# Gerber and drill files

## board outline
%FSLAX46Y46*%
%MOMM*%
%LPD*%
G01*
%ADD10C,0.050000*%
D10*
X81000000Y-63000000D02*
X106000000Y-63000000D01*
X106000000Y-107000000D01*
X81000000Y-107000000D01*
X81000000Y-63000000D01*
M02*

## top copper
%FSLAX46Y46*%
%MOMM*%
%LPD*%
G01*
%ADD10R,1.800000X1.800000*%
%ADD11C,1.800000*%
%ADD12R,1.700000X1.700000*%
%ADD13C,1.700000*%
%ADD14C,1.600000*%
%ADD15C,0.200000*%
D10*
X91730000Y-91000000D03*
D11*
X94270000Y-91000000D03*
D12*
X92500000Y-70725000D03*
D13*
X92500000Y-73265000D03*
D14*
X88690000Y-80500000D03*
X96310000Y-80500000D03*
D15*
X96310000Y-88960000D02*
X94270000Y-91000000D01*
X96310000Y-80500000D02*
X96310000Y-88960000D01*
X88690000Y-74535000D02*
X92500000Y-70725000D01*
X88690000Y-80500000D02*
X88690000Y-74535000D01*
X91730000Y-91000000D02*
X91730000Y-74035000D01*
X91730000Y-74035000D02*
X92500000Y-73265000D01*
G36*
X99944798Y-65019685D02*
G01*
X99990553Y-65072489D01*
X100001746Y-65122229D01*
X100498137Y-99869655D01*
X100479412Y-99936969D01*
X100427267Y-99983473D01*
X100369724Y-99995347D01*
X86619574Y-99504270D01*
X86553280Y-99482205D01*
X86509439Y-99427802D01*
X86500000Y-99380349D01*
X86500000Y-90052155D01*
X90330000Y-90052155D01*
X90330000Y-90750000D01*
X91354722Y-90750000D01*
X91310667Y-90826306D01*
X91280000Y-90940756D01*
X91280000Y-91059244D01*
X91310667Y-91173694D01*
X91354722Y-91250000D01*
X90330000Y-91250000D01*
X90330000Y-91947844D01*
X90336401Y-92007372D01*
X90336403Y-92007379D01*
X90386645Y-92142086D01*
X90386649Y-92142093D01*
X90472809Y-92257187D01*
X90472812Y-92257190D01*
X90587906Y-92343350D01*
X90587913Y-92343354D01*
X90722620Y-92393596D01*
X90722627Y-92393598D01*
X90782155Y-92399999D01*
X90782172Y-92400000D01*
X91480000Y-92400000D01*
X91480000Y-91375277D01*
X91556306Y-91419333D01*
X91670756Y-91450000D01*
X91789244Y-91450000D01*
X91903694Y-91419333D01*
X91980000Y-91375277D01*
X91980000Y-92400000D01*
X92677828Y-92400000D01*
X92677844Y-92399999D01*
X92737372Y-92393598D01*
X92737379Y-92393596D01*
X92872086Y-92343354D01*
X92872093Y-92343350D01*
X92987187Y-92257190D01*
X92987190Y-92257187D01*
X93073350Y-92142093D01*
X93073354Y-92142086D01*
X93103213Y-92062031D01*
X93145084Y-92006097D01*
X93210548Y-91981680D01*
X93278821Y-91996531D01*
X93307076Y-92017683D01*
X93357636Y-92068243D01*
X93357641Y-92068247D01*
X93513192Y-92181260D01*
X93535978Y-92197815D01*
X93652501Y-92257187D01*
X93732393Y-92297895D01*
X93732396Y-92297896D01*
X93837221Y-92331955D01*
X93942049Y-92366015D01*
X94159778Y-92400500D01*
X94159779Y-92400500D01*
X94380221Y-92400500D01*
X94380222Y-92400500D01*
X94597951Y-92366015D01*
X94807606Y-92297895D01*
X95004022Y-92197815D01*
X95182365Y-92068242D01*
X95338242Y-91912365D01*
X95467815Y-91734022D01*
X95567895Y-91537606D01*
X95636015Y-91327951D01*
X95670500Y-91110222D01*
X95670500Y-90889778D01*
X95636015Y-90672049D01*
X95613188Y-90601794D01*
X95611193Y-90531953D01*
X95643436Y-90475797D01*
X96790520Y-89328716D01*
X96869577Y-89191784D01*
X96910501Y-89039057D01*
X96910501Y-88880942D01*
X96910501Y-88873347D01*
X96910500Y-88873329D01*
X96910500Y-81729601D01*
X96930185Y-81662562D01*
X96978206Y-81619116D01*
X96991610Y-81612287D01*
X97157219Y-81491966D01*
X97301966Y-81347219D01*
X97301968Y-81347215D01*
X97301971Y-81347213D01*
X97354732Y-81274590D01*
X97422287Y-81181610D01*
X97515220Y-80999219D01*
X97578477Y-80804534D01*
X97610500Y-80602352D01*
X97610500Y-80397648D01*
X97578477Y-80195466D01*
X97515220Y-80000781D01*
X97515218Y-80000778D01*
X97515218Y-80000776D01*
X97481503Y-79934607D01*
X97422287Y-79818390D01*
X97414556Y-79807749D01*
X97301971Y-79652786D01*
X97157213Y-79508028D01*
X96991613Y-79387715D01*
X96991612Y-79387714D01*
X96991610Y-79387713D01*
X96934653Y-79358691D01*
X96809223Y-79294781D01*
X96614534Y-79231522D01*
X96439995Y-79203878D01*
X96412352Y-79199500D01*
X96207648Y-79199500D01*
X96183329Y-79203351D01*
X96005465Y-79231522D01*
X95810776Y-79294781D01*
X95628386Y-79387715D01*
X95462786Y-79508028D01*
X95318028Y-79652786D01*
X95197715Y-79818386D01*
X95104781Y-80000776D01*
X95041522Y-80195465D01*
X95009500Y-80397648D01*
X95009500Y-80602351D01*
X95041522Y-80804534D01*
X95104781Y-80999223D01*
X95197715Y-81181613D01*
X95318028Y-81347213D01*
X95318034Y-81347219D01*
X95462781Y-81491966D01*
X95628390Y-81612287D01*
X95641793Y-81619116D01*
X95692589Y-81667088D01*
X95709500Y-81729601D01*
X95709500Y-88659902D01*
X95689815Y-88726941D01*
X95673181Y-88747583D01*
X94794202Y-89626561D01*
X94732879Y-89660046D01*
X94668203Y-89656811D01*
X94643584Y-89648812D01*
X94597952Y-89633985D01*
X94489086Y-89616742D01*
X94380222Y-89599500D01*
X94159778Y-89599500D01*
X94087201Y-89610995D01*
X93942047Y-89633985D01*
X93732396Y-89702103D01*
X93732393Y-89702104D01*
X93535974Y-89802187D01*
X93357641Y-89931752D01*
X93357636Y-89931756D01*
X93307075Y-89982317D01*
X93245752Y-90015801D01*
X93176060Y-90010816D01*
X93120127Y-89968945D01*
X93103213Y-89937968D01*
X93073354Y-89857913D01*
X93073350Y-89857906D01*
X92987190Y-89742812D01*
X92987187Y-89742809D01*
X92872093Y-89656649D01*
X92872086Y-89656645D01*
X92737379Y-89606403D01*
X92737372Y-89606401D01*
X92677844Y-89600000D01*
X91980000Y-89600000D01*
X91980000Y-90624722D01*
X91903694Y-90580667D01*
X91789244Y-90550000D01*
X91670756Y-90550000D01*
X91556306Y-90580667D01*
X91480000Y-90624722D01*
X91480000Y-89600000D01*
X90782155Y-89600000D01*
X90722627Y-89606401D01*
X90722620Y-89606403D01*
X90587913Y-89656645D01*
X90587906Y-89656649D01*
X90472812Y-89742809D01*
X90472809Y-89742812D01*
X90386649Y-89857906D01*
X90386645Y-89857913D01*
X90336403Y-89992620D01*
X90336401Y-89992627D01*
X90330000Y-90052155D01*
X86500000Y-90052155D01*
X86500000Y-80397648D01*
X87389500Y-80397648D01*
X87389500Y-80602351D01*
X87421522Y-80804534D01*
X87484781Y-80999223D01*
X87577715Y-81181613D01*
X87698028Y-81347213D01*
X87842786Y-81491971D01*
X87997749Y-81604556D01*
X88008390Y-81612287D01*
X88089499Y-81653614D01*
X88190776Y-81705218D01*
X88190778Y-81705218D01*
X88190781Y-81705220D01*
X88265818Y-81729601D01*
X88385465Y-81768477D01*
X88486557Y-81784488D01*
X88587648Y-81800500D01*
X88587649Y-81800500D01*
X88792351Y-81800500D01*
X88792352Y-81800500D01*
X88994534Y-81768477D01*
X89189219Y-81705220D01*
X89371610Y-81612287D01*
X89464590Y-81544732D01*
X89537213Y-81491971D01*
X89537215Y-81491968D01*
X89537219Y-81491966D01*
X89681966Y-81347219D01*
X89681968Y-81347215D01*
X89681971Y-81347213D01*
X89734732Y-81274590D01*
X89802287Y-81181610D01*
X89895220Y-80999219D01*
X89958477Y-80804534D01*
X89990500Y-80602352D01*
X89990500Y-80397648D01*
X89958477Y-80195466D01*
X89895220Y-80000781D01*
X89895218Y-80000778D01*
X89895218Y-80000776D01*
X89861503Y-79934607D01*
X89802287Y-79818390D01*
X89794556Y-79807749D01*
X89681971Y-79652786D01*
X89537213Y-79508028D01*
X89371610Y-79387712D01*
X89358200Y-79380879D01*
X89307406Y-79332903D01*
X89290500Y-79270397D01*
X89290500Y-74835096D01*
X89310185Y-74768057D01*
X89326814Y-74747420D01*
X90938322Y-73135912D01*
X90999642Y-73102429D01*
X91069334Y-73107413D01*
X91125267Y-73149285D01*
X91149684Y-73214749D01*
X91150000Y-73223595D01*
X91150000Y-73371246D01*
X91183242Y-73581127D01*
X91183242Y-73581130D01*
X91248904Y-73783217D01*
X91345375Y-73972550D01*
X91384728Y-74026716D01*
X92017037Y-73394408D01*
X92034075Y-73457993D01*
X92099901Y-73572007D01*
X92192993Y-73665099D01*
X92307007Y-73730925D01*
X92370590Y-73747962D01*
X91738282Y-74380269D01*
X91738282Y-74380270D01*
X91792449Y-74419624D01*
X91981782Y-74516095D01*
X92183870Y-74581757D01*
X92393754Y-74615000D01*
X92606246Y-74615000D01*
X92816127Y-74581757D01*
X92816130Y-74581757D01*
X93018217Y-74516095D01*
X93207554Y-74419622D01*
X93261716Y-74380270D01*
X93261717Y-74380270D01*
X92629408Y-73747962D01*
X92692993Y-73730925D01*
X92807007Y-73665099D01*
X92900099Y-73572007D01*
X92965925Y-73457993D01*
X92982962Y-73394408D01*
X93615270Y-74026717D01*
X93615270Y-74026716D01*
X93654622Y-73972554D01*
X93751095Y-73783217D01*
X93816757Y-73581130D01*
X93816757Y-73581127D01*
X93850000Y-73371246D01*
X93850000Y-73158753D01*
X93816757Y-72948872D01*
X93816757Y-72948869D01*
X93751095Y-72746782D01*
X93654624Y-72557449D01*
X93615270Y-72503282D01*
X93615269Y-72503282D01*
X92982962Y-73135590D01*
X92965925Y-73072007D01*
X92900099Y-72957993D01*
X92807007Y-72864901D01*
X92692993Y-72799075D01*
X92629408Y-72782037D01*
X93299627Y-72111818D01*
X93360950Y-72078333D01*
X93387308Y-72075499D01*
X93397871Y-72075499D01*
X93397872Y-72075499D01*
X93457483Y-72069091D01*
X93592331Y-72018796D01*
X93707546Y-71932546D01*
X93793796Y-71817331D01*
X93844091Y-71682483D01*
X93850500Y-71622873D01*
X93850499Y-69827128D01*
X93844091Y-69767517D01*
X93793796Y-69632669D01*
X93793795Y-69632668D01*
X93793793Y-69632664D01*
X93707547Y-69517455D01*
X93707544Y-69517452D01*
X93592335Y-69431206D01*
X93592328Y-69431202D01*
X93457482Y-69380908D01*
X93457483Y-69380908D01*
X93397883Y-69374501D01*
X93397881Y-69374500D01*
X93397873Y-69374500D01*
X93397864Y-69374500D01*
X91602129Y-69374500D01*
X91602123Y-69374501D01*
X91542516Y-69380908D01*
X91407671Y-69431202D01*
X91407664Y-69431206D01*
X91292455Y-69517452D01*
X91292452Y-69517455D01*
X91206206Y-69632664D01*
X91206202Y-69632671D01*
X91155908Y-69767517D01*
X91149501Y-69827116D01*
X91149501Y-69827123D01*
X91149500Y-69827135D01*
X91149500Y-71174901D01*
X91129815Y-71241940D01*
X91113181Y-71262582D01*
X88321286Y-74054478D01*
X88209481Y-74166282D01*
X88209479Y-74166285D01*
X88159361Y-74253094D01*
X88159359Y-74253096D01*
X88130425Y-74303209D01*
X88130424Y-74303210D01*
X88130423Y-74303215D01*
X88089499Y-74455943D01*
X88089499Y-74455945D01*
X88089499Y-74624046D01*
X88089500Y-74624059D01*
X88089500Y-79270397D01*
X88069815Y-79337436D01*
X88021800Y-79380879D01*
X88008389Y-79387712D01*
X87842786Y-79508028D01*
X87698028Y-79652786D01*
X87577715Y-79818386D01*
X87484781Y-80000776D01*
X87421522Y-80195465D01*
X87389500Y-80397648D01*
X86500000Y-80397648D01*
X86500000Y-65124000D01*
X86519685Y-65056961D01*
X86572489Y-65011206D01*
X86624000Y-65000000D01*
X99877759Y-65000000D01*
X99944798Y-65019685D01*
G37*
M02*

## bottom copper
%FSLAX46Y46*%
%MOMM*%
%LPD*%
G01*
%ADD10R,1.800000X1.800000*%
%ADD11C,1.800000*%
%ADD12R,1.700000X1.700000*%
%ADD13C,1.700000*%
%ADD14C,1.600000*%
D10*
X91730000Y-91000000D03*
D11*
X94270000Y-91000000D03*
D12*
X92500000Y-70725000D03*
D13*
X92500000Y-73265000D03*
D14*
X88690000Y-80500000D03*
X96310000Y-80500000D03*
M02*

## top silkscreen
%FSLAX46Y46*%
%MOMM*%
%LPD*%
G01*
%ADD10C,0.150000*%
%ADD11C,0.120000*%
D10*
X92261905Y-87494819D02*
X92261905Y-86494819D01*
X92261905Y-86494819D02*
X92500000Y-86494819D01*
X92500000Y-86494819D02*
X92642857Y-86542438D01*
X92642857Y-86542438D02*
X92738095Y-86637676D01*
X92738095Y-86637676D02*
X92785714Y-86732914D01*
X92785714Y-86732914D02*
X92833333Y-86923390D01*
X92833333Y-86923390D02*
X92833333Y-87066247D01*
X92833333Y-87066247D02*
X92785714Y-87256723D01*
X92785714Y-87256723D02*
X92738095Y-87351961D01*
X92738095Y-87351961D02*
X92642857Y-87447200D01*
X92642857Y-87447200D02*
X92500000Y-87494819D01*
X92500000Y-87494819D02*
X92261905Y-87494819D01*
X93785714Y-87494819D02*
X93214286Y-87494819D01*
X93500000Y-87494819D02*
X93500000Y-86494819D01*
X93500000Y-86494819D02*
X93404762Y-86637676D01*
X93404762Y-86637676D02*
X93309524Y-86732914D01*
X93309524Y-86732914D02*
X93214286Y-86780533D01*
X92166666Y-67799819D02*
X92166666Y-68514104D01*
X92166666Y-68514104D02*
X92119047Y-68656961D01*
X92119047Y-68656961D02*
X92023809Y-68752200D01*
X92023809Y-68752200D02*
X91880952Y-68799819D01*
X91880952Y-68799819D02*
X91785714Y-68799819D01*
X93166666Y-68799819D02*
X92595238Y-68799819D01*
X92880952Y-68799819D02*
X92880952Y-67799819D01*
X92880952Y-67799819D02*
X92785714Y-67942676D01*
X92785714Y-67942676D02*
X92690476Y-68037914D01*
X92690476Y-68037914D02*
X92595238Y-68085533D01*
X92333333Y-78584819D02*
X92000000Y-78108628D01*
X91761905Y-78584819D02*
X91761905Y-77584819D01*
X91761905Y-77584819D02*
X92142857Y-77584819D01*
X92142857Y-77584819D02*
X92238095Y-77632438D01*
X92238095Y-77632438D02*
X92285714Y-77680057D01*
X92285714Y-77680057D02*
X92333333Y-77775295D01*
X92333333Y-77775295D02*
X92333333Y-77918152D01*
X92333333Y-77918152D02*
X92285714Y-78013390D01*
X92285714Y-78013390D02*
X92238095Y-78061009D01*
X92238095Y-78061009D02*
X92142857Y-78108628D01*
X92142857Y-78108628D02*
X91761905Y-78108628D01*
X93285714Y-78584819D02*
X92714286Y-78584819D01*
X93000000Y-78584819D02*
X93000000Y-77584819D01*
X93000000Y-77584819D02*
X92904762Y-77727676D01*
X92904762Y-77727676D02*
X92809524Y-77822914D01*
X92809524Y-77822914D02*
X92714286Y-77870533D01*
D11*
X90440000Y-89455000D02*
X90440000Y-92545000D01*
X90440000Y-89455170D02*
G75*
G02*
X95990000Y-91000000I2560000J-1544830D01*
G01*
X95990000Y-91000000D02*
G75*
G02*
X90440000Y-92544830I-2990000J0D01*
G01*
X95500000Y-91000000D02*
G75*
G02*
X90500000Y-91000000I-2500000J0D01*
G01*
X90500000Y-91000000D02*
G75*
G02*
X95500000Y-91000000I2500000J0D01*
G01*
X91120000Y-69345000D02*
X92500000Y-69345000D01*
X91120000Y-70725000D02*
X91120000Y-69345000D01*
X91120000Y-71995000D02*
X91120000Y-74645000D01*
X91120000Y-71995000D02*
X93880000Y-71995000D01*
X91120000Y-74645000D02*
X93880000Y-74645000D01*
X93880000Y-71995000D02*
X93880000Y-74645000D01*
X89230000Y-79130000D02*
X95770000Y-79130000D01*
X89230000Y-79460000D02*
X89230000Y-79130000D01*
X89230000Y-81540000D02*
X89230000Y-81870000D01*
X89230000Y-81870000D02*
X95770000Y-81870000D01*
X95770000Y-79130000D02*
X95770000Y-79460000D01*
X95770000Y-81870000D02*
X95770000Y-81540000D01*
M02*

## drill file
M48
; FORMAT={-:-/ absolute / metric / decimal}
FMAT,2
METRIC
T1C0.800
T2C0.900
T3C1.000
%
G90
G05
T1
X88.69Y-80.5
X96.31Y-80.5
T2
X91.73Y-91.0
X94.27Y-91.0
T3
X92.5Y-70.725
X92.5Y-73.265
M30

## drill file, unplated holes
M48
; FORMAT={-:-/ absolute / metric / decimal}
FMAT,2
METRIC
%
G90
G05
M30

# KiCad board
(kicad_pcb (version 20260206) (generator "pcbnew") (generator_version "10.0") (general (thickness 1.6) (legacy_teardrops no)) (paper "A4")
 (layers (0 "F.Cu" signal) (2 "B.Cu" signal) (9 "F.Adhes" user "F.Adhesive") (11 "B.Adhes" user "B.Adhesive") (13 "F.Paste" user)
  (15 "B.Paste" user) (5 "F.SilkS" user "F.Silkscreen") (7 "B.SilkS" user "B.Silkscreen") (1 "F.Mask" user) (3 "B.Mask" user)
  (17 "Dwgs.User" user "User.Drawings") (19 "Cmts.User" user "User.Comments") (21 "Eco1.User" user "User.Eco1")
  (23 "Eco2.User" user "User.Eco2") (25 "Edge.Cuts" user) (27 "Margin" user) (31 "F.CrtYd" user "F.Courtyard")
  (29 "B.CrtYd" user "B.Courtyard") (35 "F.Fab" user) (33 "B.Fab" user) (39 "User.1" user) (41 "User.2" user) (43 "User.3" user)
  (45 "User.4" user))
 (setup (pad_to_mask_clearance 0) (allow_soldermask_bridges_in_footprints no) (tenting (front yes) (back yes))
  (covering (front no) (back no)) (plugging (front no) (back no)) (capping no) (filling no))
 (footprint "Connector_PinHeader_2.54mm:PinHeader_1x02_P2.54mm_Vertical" (layer "F.Cu") (at 92.5 70.725)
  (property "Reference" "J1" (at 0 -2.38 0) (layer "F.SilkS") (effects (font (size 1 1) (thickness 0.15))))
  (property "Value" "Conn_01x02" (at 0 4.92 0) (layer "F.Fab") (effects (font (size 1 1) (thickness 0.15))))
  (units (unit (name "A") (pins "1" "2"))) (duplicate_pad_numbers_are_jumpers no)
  (fp_line (start -1.38 -1.38) (end 0 -1.38) (stroke (width 0.12) (type solid)) (layer "F.SilkS"))
  (fp_line (start -1.38 0) (end -1.38 -1.38) (stroke (width 0.12) (type solid)) (layer "F.SilkS"))
  (fp_line (start -1.38 1.27) (end -1.38 3.92) (stroke (width 0.12) (type solid)) (layer "F.SilkS"))
  (fp_line (start -1.38 1.27) (end 1.38 1.27) (stroke (width 0.12) (type solid)) (layer "F.SilkS"))
  (fp_line (start -1.38 3.92) (end 1.38 3.92) (stroke (width 0.12) (type solid)) (layer "F.SilkS"))
  (fp_line (start 1.38 1.27) (end 1.38 3.92) (stroke (width 0.12) (type solid)) (layer "F.SilkS"))
  (pad "1" thru_hole rect (at 0 0) (size 1.7 1.7) (drill 1) (layers "*.Cu" "*.Mask") (remove_unused_layers no) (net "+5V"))
  (pad "2" thru_hole circle (at 0 2.54) (size 1.7 1.7) (drill 1) (layers "*.Cu" "*.Mask") (remove_unused_layers no) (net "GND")))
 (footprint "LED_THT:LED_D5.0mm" (layer "F.Cu") (at 91.73 91)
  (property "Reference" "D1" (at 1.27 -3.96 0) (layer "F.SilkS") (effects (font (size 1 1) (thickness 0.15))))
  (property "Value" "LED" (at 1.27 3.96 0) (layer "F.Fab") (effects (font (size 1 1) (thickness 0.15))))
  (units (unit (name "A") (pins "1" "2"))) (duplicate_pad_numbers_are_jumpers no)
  (fp_line (start -1.29 -1.545) (end -1.29 1.545) (stroke (width 0.12) (type solid)) (layer "F.SilkS"))
  (fp_arc (start -1.29 -1.54483) (mid 2.071779 -2.880495) (end 4.26 0) (stroke (width 0.12) (type solid)) (layer "F.SilkS"))
  (fp_arc (start 4.26 0) (mid 2.071779 2.880495) (end -1.29 1.54483) (stroke (width 0.12) (type solid)) (layer "F.SilkS"))
  (fp_circle (center 1.27 0) (end 3.77 0) (stroke (width 0.12) (type solid)) (fill no) (layer "F.SilkS"))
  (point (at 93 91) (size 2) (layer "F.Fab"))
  (pad "1" thru_hole rect (at 0 0) (size 1.8 1.8) (drill 0.9) (layers "*.Cu" "*.Mask") (remove_unused_layers no) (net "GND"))
  (pad "2" thru_hole circle (at 2.54 0) (size 1.8 1.8) (drill 0.9) (layers "*.Cu" "*.Mask") (remove_unused_layers no) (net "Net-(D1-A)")))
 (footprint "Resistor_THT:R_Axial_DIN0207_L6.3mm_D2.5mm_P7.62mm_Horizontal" (layer "F.Cu") (at 88.69 80.5)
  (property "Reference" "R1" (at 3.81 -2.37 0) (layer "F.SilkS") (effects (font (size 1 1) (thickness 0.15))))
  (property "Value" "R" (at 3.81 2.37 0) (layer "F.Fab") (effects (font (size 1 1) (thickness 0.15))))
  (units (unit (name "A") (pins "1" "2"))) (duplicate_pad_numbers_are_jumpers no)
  (fp_line (start 0.54 -1.37) (end 7.08 -1.37) (stroke (width 0.12) (type solid)) (layer "F.SilkS"))
  (fp_line (start 0.54 -1.04) (end 0.54 -1.37) (stroke (width 0.12) (type solid)) (layer "F.SilkS"))
  (fp_line (start 0.54 1.04) (end 0.54 1.37) (stroke (width 0.12) (type solid)) (layer "F.SilkS"))
  (fp_line (start 0.54 1.37) (end 7.08 1.37) (stroke (width 0.12) (type solid)) (layer "F.SilkS"))
  (fp_line (start 7.08 -1.37) (end 7.08 -1.04) (stroke (width 0.12) (type solid)) (layer "F.SilkS"))
  (fp_line (start 7.08 1.37) (end 7.08 1.04) (stroke (width 0.12) (type solid)) (layer "F.SilkS"))
  (pad "1" thru_hole circle (at 0 0) (size 1.6 1.6) (drill 0.8) (layers "*.Cu" "*.Mask") (remove_unused_layers no) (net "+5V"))
  (pad "2" thru_hole circle (at 7.62 0) (size 1.6 1.6) (drill 0.8) (layers "*.Cu" "*.Mask") (remove_unused_layers no) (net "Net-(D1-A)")))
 (gr_rect (start 81 63) (end 106 107) (stroke (width 0.05) (type default)) (fill no) (layer "Edge.Cuts"))
 (segment (start 91.73 74.035) (end 92.5 73.265) (width 0.2) (layer "F.Cu") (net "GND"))
 (segment (start 91.73 91) (end 91.73 74.035) (width 0.2) (layer "F.Cu") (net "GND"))
 (segment (start 88.69 74.535) (end 92.5 70.725) (width 0.2) (layer "F.Cu") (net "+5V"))
 (segment (start 88.69 80.5) (end 88.69 74.535) (width 0.2) (layer "F.Cu") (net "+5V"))
 (segment (start 96.31 80.5) (end 96.31 88.96) (width 0.2) (layer "F.Cu") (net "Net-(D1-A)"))
 (segment (start 96.31 88.96) (end 94.27 91) (width 0.2) (layer "F.Cu") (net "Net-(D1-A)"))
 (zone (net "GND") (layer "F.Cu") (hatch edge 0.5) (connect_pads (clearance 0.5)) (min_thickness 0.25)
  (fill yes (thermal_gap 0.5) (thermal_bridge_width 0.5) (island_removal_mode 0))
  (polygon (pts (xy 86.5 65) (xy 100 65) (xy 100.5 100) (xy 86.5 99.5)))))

